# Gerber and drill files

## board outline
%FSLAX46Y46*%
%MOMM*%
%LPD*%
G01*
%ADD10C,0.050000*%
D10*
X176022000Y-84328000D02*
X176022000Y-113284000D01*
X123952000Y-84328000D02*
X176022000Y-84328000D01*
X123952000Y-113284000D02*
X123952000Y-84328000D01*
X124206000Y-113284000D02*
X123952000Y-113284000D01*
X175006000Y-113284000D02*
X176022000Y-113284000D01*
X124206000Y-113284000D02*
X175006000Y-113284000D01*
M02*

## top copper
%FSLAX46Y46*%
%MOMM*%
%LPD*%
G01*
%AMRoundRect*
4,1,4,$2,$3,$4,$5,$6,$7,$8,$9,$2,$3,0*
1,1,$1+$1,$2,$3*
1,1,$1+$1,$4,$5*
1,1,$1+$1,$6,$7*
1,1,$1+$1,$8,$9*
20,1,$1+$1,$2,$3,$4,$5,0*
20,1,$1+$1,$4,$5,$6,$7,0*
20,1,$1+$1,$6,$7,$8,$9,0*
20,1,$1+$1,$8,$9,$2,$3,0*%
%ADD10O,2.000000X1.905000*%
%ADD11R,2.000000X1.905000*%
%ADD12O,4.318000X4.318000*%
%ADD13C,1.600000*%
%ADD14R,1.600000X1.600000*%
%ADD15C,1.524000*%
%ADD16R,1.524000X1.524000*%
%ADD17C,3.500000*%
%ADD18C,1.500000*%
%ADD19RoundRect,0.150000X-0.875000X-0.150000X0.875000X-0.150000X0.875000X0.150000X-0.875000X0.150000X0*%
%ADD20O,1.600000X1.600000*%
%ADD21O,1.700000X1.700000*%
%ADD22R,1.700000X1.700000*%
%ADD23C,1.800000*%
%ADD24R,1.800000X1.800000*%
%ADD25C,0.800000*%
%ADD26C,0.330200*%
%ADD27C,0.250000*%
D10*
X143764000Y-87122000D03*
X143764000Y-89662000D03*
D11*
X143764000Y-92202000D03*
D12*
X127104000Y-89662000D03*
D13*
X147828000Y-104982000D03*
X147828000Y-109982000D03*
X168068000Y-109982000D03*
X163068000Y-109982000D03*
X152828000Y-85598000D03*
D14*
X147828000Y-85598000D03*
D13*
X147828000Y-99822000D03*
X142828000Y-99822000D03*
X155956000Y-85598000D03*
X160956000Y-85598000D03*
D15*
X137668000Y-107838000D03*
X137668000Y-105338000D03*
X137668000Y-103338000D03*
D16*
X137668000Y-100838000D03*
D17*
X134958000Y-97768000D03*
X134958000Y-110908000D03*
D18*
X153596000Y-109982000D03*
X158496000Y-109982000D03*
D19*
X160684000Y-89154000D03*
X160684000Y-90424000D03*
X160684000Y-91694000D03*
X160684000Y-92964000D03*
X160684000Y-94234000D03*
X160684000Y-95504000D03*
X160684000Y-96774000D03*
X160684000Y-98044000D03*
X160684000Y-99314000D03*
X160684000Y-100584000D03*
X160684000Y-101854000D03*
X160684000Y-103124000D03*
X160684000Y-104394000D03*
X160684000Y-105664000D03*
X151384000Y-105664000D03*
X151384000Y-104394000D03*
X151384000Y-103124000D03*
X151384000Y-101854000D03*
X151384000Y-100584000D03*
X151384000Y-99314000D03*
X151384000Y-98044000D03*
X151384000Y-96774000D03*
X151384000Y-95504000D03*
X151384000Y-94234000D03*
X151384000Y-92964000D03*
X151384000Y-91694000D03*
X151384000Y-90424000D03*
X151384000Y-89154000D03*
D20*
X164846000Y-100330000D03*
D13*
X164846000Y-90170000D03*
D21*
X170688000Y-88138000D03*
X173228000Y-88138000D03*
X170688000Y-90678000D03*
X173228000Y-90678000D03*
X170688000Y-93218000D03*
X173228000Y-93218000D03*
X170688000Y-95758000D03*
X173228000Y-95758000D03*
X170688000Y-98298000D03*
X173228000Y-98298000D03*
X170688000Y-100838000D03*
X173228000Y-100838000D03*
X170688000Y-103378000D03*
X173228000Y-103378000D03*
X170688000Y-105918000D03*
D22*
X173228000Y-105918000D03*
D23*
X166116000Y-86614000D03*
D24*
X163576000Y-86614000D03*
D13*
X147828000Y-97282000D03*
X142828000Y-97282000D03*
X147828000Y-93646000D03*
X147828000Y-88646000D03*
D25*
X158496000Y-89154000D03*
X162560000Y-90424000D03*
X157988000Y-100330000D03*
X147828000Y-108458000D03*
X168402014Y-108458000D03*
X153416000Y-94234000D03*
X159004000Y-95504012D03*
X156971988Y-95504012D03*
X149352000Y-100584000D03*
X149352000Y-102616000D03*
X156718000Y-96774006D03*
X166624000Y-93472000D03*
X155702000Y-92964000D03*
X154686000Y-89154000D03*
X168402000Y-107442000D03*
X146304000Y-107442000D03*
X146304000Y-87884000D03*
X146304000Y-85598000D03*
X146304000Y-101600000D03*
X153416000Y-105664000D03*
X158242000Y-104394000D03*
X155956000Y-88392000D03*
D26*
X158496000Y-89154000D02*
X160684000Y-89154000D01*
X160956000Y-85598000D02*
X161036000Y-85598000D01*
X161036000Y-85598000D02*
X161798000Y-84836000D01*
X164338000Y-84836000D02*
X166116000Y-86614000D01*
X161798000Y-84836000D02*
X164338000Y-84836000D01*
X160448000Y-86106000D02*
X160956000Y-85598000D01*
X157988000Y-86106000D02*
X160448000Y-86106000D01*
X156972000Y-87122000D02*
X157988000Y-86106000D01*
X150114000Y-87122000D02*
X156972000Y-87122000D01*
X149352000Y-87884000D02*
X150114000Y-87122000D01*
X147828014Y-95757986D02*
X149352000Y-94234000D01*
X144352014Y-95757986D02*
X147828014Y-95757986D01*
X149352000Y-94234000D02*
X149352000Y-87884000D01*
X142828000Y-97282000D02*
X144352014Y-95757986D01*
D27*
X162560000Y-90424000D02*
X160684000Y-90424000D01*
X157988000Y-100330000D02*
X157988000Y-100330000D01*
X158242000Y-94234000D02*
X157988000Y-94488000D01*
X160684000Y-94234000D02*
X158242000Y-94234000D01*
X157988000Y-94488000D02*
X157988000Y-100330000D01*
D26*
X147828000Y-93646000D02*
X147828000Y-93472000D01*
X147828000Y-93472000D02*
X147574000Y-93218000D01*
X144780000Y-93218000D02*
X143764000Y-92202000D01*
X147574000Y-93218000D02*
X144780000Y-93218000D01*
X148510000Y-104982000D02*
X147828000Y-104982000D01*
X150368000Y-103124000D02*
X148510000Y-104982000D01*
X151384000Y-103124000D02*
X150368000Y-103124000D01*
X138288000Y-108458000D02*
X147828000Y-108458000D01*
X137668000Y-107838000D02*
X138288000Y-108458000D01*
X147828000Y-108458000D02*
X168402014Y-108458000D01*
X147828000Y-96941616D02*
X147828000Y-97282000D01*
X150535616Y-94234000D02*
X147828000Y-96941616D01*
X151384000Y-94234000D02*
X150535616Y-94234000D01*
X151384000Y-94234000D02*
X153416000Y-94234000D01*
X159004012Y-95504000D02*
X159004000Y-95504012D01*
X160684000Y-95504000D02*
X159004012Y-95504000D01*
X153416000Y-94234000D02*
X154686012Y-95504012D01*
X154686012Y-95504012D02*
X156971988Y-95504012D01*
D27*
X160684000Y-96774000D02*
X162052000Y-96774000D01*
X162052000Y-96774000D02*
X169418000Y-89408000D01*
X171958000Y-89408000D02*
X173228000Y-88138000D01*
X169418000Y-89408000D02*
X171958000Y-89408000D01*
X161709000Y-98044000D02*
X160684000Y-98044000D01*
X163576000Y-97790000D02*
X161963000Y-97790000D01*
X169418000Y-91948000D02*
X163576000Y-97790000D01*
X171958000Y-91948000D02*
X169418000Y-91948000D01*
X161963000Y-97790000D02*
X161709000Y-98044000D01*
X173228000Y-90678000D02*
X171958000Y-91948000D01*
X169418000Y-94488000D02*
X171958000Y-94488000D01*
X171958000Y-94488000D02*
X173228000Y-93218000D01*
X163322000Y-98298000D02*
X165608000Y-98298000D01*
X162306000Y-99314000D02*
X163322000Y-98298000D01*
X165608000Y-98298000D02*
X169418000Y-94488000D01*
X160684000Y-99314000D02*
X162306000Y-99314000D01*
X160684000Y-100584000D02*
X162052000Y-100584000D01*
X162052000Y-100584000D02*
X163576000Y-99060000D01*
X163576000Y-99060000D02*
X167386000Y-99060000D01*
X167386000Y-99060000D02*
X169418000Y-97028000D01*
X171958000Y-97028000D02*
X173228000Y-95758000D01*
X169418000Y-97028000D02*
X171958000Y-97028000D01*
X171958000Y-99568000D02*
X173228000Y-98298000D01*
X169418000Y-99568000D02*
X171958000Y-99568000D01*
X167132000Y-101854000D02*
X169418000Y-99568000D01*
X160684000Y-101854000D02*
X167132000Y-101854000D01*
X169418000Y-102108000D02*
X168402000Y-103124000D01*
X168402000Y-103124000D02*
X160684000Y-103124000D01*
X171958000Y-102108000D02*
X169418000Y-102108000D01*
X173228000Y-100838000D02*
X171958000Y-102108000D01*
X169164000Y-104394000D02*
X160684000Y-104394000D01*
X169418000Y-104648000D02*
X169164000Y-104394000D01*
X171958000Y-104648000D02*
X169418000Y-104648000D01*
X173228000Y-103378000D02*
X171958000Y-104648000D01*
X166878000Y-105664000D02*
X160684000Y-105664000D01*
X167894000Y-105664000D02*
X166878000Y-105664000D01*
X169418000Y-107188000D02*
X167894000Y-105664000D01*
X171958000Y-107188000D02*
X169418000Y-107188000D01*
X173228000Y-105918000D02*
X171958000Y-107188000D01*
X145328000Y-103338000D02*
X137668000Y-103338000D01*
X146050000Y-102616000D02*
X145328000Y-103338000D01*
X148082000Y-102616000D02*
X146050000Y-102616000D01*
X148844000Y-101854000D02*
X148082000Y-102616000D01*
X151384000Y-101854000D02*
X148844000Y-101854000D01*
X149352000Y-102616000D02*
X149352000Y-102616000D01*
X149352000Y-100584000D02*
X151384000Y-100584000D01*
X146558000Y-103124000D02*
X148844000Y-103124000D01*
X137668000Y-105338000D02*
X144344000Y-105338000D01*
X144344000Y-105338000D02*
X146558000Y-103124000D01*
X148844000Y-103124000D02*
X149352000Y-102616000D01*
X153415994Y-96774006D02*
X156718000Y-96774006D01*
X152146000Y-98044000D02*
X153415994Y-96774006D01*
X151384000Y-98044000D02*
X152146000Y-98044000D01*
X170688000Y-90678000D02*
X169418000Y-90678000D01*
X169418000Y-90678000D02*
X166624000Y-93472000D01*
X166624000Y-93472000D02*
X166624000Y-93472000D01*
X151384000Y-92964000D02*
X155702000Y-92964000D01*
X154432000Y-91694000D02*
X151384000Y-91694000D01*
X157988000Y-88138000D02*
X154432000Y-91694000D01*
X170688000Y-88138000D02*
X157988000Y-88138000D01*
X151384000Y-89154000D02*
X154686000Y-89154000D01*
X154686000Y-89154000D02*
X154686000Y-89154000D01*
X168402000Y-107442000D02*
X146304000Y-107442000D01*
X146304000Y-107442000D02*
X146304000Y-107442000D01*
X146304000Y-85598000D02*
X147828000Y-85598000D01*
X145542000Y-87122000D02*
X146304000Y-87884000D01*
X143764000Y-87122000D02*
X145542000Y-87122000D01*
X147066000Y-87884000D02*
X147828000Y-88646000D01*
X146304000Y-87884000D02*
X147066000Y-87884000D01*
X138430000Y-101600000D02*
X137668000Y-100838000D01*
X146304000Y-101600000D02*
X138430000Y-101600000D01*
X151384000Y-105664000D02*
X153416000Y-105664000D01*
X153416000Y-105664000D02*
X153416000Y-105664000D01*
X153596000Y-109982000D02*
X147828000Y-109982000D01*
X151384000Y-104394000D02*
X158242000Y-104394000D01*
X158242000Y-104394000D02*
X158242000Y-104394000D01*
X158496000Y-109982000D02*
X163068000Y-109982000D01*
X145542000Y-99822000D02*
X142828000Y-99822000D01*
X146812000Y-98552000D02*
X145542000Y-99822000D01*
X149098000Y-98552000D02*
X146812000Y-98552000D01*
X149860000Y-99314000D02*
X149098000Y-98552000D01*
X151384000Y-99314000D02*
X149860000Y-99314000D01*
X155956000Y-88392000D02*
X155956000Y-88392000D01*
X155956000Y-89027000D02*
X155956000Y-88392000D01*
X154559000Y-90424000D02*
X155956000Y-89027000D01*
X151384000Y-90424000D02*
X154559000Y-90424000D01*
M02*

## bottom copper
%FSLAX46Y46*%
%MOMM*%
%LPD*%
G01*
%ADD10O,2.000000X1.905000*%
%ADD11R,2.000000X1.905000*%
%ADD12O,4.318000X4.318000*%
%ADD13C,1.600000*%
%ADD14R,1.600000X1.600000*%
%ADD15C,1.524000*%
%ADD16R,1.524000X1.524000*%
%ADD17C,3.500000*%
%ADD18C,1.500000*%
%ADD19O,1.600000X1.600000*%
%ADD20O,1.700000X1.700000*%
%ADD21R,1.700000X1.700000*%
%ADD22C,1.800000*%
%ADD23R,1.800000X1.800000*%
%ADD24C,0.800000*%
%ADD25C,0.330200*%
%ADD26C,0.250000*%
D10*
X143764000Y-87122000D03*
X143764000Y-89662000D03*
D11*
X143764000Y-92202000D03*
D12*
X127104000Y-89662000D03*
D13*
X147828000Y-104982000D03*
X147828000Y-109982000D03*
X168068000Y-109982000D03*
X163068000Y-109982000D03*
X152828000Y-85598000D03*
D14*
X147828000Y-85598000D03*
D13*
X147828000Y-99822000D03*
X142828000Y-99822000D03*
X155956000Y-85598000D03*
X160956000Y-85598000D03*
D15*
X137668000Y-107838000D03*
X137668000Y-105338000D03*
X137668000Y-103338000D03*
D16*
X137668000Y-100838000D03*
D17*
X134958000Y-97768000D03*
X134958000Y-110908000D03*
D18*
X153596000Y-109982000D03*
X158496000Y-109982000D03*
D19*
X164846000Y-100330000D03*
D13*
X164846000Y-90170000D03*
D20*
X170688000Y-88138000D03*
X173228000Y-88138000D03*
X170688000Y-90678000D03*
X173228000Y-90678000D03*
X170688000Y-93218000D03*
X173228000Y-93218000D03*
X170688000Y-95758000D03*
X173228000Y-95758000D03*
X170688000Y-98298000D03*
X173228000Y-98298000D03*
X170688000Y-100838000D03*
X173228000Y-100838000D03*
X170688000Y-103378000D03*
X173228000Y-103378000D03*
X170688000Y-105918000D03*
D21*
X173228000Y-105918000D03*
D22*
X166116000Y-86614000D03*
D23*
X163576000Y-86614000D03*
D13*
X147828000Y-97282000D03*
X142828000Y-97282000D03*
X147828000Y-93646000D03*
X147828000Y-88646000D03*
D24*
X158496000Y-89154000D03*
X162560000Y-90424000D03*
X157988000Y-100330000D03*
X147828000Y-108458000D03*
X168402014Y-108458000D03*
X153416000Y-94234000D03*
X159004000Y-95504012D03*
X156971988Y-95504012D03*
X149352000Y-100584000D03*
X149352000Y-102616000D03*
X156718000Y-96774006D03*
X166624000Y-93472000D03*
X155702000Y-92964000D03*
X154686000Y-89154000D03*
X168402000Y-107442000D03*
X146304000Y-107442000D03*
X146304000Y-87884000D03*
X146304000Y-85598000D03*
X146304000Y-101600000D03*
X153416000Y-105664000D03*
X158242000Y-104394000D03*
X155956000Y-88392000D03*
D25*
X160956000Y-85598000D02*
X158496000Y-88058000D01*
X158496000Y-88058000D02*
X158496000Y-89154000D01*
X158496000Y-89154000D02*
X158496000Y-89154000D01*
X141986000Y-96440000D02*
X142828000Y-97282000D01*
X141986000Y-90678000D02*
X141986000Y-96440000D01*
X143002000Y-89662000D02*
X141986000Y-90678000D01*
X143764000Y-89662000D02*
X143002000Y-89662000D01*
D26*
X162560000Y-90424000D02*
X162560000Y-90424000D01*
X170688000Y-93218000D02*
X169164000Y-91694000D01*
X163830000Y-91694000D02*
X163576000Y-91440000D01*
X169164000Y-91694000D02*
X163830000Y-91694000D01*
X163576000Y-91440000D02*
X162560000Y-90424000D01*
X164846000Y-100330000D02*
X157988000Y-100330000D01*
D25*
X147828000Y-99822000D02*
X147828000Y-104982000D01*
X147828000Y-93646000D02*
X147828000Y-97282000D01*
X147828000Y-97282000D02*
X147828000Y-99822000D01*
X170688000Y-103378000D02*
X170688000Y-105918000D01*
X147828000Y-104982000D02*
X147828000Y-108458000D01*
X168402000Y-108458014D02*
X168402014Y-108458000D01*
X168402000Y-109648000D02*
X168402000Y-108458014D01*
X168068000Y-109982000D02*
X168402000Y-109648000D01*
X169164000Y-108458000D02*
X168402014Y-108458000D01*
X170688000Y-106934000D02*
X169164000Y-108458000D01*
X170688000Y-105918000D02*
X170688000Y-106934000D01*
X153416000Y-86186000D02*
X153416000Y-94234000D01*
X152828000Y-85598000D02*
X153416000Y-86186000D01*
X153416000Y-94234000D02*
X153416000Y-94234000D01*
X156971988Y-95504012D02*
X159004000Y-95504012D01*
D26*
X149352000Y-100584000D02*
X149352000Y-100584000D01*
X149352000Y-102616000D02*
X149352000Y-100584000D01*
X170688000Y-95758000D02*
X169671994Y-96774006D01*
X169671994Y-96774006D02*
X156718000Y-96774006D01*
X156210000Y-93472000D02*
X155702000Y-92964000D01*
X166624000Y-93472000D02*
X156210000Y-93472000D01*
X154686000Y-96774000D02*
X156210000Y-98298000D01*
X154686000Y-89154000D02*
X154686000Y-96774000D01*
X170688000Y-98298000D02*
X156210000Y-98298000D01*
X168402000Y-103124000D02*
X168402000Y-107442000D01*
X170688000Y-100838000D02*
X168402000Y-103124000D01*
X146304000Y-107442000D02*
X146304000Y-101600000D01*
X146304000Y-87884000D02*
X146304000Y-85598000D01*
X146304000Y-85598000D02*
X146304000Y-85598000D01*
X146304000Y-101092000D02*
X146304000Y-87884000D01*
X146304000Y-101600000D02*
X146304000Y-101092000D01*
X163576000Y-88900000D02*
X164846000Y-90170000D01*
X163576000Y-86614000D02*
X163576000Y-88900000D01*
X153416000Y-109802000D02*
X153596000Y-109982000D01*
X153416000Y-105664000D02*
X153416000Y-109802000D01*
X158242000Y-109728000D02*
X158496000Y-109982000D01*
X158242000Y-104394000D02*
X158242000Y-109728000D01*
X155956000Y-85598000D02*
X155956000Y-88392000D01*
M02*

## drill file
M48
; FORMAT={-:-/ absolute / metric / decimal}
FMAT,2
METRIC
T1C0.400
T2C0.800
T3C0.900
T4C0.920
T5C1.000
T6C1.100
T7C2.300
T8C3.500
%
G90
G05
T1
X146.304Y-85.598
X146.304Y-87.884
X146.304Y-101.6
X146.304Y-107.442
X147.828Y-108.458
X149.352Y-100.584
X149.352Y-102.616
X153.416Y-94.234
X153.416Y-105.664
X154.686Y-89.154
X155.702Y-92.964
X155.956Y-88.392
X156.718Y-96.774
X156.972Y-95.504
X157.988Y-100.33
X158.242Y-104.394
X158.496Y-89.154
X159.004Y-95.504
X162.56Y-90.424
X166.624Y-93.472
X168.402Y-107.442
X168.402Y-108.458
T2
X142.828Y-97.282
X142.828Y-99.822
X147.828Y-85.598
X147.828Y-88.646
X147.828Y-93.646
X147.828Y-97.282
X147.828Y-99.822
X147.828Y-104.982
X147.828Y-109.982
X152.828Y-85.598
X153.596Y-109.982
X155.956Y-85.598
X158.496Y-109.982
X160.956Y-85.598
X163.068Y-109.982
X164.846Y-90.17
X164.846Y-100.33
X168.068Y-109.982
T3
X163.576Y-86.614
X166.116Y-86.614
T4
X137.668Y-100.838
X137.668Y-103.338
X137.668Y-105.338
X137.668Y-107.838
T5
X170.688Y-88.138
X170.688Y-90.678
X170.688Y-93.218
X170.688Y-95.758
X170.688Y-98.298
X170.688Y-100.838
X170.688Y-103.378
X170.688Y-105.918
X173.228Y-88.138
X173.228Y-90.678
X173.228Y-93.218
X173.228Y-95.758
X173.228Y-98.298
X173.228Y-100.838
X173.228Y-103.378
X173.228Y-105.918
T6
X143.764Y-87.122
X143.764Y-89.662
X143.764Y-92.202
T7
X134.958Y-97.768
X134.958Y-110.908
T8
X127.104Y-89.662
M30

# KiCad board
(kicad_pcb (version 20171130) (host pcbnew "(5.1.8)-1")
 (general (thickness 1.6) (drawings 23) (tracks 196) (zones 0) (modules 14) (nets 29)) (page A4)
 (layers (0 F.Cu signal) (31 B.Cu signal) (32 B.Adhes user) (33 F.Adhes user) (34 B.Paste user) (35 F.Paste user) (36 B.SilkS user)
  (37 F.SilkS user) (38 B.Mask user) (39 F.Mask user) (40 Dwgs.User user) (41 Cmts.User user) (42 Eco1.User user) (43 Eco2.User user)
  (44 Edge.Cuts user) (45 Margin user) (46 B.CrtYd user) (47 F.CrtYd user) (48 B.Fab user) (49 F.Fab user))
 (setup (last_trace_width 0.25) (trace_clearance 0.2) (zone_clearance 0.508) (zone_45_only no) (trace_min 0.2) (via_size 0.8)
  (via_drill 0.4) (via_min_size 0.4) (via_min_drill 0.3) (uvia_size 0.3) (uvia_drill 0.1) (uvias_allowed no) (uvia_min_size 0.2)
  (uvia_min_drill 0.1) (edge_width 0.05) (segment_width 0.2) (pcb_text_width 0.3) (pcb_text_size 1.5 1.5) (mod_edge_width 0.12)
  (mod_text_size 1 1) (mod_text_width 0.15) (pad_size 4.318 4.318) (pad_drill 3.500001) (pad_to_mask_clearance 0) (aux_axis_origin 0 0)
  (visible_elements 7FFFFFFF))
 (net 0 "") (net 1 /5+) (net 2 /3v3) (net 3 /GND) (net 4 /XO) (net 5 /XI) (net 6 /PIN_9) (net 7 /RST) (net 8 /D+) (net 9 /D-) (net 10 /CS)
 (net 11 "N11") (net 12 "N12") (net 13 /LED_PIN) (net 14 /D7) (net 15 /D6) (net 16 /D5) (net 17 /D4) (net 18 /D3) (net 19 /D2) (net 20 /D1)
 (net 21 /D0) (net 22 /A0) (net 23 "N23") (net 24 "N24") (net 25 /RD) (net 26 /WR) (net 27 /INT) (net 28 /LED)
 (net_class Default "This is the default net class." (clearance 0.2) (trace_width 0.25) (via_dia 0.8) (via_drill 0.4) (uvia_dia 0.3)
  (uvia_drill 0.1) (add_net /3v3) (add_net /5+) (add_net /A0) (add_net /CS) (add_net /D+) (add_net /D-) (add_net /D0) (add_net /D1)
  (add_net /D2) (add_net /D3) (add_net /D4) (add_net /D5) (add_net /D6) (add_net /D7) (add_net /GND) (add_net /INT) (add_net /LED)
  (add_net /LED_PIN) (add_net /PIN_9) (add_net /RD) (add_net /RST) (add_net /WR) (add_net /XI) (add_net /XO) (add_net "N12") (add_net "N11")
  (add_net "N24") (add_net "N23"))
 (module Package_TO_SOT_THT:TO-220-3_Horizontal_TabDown (layer F.Cu) (at 143.764 92.202 90)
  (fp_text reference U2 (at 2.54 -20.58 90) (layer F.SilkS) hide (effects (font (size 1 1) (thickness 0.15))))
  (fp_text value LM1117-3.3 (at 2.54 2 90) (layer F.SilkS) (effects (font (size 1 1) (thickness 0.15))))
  (pad 3 thru_hole oval (at 5.08 0 90) (size 1.905 2) (drill 1.1) (layers *.Cu *.Mask) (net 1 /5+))
  (pad 2 thru_hole oval (at 2.54 0 90) (size 1.905 2) (drill 1.1) (layers *.Cu *.Mask) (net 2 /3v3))
  (pad 1 thru_hole rect (at 0 0 90) (size 1.905 2) (drill 1.1) (layers *.Cu *.Mask) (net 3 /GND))
  (pad "" thru_hole oval (at 2.54 -16.66 90) (size 4.318 4.318) (drill 3.500001) (layers *.Cu *.Mask)))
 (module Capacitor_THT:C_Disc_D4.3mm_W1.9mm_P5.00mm (layer F.Cu) (at 147.828 109.982 90)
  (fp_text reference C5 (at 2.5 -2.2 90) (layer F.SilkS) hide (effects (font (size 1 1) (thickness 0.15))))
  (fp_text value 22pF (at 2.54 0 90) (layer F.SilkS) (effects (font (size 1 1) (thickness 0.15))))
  (pad 2 thru_hole circle (at 5 0 90) (size 1.6 1.6) (drill 0.8) (layers *.Cu *.Mask) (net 3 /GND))
  (pad 1 thru_hole circle (at 0 0 90) (size 1.6 1.6) (drill 0.8) (layers *.Cu *.Mask) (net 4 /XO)))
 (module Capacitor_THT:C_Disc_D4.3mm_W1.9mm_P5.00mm (layer F.Cu) (at 163.068 109.982)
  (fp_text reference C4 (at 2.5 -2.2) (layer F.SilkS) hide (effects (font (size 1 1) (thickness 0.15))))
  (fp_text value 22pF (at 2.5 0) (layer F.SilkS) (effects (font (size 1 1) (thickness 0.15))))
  (pad 2 thru_hole circle (at 5 0) (size 1.6 1.6) (drill 0.8) (layers *.Cu *.Mask) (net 3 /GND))
  (pad 1 thru_hole circle (at 0 0) (size 1.6 1.6) (drill 0.8) (layers *.Cu *.Mask) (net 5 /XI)))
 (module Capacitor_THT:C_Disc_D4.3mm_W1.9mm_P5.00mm (layer F.Cu) (at 147.828 85.598)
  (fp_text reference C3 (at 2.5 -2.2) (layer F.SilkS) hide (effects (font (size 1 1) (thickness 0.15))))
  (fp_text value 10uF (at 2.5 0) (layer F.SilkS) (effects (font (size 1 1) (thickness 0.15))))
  (pad 2 thru_hole circle (at 5 0) (size 1.6 1.6) (drill 0.8) (layers *.Cu *.Mask) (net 3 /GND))
  (pad 1 thru_hole rect (at 0 0) (size 1.6 1.6) (drill 0.8) (layers *.Cu *.Mask) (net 1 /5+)))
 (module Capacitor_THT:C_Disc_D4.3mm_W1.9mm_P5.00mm (layer F.Cu) (at 142.828 99.822)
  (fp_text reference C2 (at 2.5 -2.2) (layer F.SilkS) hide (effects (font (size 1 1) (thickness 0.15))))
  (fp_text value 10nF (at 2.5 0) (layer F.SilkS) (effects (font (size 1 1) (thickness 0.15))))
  (pad 2 thru_hole circle (at 5 0) (size 1.6 1.6) (drill 0.8) (layers *.Cu *.Mask) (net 3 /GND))
  (pad 1 thru_hole circle (at 0 0) (size 1.6 1.6) (drill 0.8) (layers *.Cu *.Mask) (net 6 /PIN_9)))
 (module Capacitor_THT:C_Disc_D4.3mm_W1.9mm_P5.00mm (layer F.Cu) (at 160.956 85.598 180)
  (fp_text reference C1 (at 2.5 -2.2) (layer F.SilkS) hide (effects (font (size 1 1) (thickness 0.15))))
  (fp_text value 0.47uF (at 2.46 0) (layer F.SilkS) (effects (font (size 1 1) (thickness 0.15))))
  (pad 2 thru_hole circle (at 5 0 180) (size 1.6 1.6) (drill 0.8) (layers *.Cu *.Mask) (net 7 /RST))
  (pad 1 thru_hole circle (at 0 0 180) (size 1.6 1.6) (drill 0.8) (layers *.Cu *.Mask) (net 2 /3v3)))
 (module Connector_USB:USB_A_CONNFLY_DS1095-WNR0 (layer F.Cu) (at 137.668 100.838 270)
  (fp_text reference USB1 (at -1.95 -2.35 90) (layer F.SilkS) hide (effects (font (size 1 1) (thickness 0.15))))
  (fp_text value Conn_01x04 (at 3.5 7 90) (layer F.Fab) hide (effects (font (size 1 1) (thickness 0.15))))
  (pad 4 thru_hole circle (at 7 0 270) (size 1.524 1.524) (drill 0.92) (layers *.Cu *.Mask) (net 3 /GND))
  (pad 3 thru_hole circle (at 4.5 0 270) (size 1.524 1.524) (drill 0.92) (layers *.Cu *.Mask) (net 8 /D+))
  (pad 2 thru_hole circle (at 2.5 0 270) (size 1.524 1.524) (drill 0.92) (layers *.Cu *.Mask) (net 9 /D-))
  (pad 1 thru_hole rect (at 0 0 270) (size 1.524 1.524) (drill 0.92) (layers *.Cu *.Mask) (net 1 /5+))
  (pad 5 thru_hole circle (at -3.07 2.71 270) (size 3.5 3.5) (drill 2.3) (layers *.Cu *.Mask))
  (pad 5 thru_hole circle (at 10.07 2.71 270) (size 3.5 3.5) (drill 2.3) (layers *.Cu *.Mask)))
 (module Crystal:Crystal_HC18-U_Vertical (layer F.Cu) (at 158.496 109.982 180)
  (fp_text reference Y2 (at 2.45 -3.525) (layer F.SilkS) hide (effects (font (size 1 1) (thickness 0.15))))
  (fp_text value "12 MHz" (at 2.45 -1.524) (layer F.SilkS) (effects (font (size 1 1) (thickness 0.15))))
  (pad 2 thru_hole circle (at 4.9 0 180) (size 1.5 1.5) (drill 0.8) (layers *.Cu *.Mask) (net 4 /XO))
  (pad 1 thru_hole circle (at 0 0 180) (size 1.5 1.5) (drill 0.8) (layers *.Cu *.Mask) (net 5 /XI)))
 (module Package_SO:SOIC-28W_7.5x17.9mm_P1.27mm (layer F.Cu) (at 156.034 97.409)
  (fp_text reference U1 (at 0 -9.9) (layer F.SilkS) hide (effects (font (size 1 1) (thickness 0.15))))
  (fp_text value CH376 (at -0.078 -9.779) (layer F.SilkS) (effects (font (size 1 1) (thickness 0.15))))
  (pad 28 smd roundrect (at 4.65 -8.255) (size 2.05 0.6) (layers F.Cu F.Paste F.Mask) (roundrect_rratio 0.25) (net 2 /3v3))
  (pad 27 smd roundrect (at 4.65 -6.985) (size 2.05 0.6) (layers F.Cu F.Paste F.Mask) (roundrect_rratio 0.25) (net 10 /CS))
  (pad 26 smd roundrect (at 4.65 -5.715) (size 2.05 0.6) (layers F.Cu F.Paste F.Mask) (roundrect_rratio 0.25) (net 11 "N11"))
  (pad 25 smd roundrect (at 4.65 -4.445) (size 2.05 0.6) (layers F.Cu F.Paste F.Mask) (roundrect_rratio 0.25) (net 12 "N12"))
  (pad 24 smd roundrect (at 4.65 -3.175) (size 2.05 0.6) (layers F.Cu F.Paste F.Mask) (roundrect_rratio 0.25) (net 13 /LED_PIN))
  (pad 23 smd roundrect (at 4.65 -1.905) (size 2.05 0.6) (layers F.Cu F.Paste F.Mask) (roundrect_rratio 0.25) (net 3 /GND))
  (pad 22 smd roundrect (at 4.65 -0.635) (size 2.05 0.6) (layers F.Cu F.Paste F.Mask) (roundrect_rratio 0.25) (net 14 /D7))
  (pad 21 smd roundrect (at 4.65 0.635) (size 2.05 0.6) (layers F.Cu F.Paste F.Mask) (roundrect_rratio 0.25) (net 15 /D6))
  (pad 20 smd roundrect (at 4.65 1.905) (size 2.05 0.6) (layers F.Cu F.Paste F.Mask) (roundrect_rratio 0.25) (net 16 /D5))
  (pad 19 smd roundrect (at 4.65 3.175) (size 2.05 0.6) (layers F.Cu F.Paste F.Mask) (roundrect_rratio 0.25) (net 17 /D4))
  (pad 18 smd roundrect (at 4.65 4.445) (size 2.05 0.6) (layers F.Cu F.Paste F.Mask) (roundrect_rratio 0.25) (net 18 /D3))
  (pad 17 smd roundrect (at 4.65 5.715) (size 2.05 0.6) (layers F.Cu F.Paste F.Mask) (roundrect_rratio 0.25) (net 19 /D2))
  (pad 16 smd roundrect (at 4.65 6.985) (size 2.05 0.6) (layers F.Cu F.Paste F.Mask) (roundrect_rratio 0.25) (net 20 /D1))
  (pad 15 smd roundrect (at 4.65 8.255) (size 2.05 0.6) (layers F.Cu F.Paste F.Mask) (roundrect_rratio 0.25) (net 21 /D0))
  (pad 14 smd roundrect (at -4.65 8.255) (size 2.05 0.6) (layers F.Cu F.Paste F.Mask) (roundrect_rratio 0.25) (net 4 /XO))
  (pad 13 smd roundrect (at -4.65 6.985) (size 2.05 0.6) (layers F.Cu F.Paste F.Mask) (roundrect_rratio 0.25) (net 5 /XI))
  (pad 12 smd roundrect (at -4.65 5.715) (size 2.05 0.6) (layers F.Cu F.Paste F.Mask) (roundrect_rratio 0.25) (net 3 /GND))
  (pad 11 smd roundrect (at -4.65 4.445) (size 2.05 0.6) (layers F.Cu F.Paste F.Mask) (roundrect_rratio 0.25) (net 9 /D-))
  (pad 10 smd roundrect (at -4.65 3.175) (size 2.05 0.6) (layers F.Cu F.Paste F.Mask) (roundrect_rratio 0.25) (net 8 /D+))
  (pad 9 smd roundrect (at -4.65 1.905) (size 2.05 0.6) (layers F.Cu F.Paste F.Mask) (roundrect_rratio 0.25) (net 6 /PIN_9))
  (pad 8 smd roundrect (at -4.65 0.635) (size 2.05 0.6) (layers F.Cu F.Paste F.Mask) (roundrect_rratio 0.25) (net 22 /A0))
  (pad 7 smd roundrect (at -4.65 -0.635) (size 2.05 0.6) (layers F.Cu F.Paste F.Mask) (roundrect_rratio 0.25) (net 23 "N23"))
  (pad 6 smd roundrect (at -4.65 -1.905) (size 2.05 0.6) (layers F.Cu F.Paste F.Mask) (roundrect_rratio 0.25) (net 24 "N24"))
  (pad 5 smd roundrect (at -4.65 -3.175) (size 2.05 0.6) (layers F.Cu F.Paste F.Mask) (roundrect_rratio 0.25) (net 3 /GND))
  (pad 4 smd roundrect (at -4.65 -4.445) (size 2.05 0.6) (layers F.Cu F.Paste F.Mask) (roundrect_rratio 0.25) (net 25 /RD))
  (pad 3 smd roundrect (at -4.65 -5.715) (size 2.05 0.6) (layers F.Cu F.Paste F.Mask) (roundrect_rratio 0.25) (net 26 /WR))
  (pad 2 smd roundrect (at -4.65 -6.985) (size 2.05 0.6) (layers F.Cu F.Paste F.Mask) (roundrect_rratio 0.25) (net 7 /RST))
  (pad 1 smd roundrect (at -4.65 -8.255) (size 2.05 0.6) (layers F.Cu F.Paste F.Mask) (roundrect_rratio 0.25) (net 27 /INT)))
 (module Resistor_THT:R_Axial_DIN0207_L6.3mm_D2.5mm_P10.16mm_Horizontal (layer F.Cu) (at 164.846 90.17 270)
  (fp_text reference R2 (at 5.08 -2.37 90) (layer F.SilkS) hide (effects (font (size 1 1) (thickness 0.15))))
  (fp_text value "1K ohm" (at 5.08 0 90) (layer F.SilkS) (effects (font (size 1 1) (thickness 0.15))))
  (pad 2 thru_hole oval (at 10.16 0 270) (size 1.6 1.6) (drill 0.8) (layers *.Cu *.Mask) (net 13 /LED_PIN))
  (pad 1 thru_hole circle (at 0 0 270) (size 1.6 1.6) (drill 0.8) (layers *.Cu *.Mask) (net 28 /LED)))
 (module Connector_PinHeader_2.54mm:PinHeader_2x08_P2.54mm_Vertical (layer F.Cu) (at 173.228 105.918 180)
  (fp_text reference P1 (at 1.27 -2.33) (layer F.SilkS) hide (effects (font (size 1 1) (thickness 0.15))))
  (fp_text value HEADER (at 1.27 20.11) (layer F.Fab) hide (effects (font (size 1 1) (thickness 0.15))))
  (pad 16 thru_hole oval (at 2.54 17.78 180) (size 1.7 1.7) (drill 1) (layers *.Cu *.Mask) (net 26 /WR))
  (pad 15 thru_hole oval (at 0 17.78 180) (size 1.7 1.7) (drill 1) (layers *.Cu *.Mask) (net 14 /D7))
  (pad 14 thru_hole oval (at 2.54 15.24 180) (size 1.7 1.7) (drill 1) (layers *.Cu *.Mask) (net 25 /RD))
  (pad 13 thru_hole oval (at 0 15.24 180) (size 1.7 1.7) (drill 1) (layers *.Cu *.Mask) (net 15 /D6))
  (pad 12 thru_hole oval (at 2.54 12.7 180) (size 1.7 1.7) (drill 1) (layers *.Cu *.Mask) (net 10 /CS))
  (pad 11 thru_hole oval (at 0 12.7 180) (size 1.7 1.7) (drill 1) (layers *.Cu *.Mask) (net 16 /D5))
  (pad 10 thru_hole oval (at 2.54 10.16 180) (size 1.7 1.7) (drill 1) (layers *.Cu *.Mask) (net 22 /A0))
  (pad 9 thru_hole oval (at 0 10.16 180) (size 1.7 1.7) (drill 1) (layers *.Cu *.Mask) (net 17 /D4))
  (pad 8 thru_hole oval (at 2.54 7.62 180) (size 1.7 1.7) (drill 1) (layers *.Cu *.Mask) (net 27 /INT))
  (pad 7 thru_hole oval (at 0 7.62 180) (size 1.7 1.7) (drill 1) (layers *.Cu *.Mask) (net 18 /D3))
  (pad 6 thru_hole oval (at 2.54 5.08 180) (size 1.7 1.7) (drill 1) (layers *.Cu *.Mask) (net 1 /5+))
  (pad 5 thru_hole oval (at 0 5.08 180) (size 1.7 1.7) (drill 1) (layers *.Cu *.Mask) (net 19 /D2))
  (pad 4 thru_hole oval (at 2.54 2.54 180) (size 1.7 1.7) (drill 1) (layers *.Cu *.Mask) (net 3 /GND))
  (pad 3 thru_hole oval (at 0 2.54 180) (size 1.7 1.7) (drill 1) (layers *.Cu *.Mask) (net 20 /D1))
  (pad 2 thru_hole oval (at 2.54 0 180) (size 1.7 1.7) (drill 1) (layers *.Cu *.Mask) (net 3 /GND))
  (pad 1 thru_hole rect (at 0 0 180) (size 1.7 1.7) (drill 1) (layers *.Cu *.Mask) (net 21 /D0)))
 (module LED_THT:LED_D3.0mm (layer F.Cu) (at 163.576 86.614)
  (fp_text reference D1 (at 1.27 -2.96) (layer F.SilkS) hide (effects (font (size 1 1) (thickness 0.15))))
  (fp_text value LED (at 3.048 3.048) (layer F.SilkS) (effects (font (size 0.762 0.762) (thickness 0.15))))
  (pad 2 thru_hole circle (at 2.54 0) (size 1.8 1.8) (drill 0.9) (layers *.Cu *.Mask) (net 2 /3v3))
  (pad 1 thru_hole rect (at 0 0) (size 1.8 1.8) (drill 0.9) (layers *.Cu *.Mask) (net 28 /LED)))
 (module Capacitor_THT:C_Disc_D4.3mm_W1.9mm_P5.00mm (layer F.Cu) (at 142.828 97.282)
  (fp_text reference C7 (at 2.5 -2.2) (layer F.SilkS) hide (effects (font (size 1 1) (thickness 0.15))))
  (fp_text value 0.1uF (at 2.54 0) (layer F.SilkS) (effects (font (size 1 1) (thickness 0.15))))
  (pad 2 thru_hole circle (at 5 0) (size 1.6 1.6) (drill 0.8) (layers *.Cu *.Mask) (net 3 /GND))
  (pad 1 thru_hole circle (at 0 0) (size 1.6 1.6) (drill 0.8) (layers *.Cu *.Mask) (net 2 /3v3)))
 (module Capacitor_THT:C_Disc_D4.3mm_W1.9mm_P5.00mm (layer F.Cu) (at 147.828 88.646 270)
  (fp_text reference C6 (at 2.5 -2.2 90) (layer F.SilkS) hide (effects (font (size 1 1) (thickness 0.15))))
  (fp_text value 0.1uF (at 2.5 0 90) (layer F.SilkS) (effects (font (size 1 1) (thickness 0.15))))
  (pad 2 thru_hole circle (at 5 0 270) (size 1.6 1.6) (drill 0.8) (layers *.Cu *.Mask) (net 3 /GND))
  (pad 1 thru_hole circle (at 0 0 270) (size 1.6 1.6) (drill 0.8) (layers *.Cu *.Mask) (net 1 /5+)))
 (gr_line (start 176.022 84.328) (end 176.022 113.284) (layer Edge.Cuts) (width 0.05))
 (gr_line (start 123.952 84.328) (end 176.022 84.328) (layer Edge.Cuts) (width 0.05))
 (gr_line (start 123.952 113.284) (end 123.952 84.328) (layer Edge.Cuts) (width 0.05))
 (gr_line (start 124.206 113.284) (end 123.952 113.284) (layer Edge.Cuts) (width 0.05))
 (gr_line (start 175.006 113.284) (end 176.022 113.284) (layer Edge.Cuts) (width 0.05))
 (gr_line (start 124.206 113.284) (end 175.006 113.284) (layer Edge.Cuts) (width 0.05))
 (segment (start 160.956 85.598) (end 158.496 88.058) (width 0.3302) (layer B.Cu) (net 2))
 (segment (start 158.496 88.058) (end 158.496 89.154) (width 0.3302) (layer B.Cu) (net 2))
 (segment (start 158.496 89.154) (end 158.496 89.154) (width 0.3302) (layer B.Cu) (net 2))
 (via (at 158.496 89.154) (size 0.8) (drill 0.4) (layers F.Cu B.Cu) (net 2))
 (segment (start 158.496 89.154) (end 160.684 89.154) (width 0.3302) (layer F.Cu) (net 2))
 (segment (start 160.956 85.598) (end 161.036 85.598) (width 0.3302) (layer F.Cu) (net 2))
 (segment (start 161.036 85.598) (end 161.798 84.836) (width 0.3302) (layer F.Cu) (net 2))
 (segment (start 164.338 84.836) (end 166.116 86.614) (width 0.3302) (layer F.Cu) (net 2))
 (segment (start 161.798 84.836) (end 164.338 84.836) (width 0.3302) (layer F.Cu) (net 2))
 (segment (start 141.986 96.44) (end 142.828 97.282) (width 0.3302) (layer B.Cu) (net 2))
 (segment (start 141.986 90.678) (end 141.986 96.44) (width 0.3302) (layer B.Cu) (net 2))
 (segment (start 143.002 89.662) (end 141.986 90.678) (width 0.3302) (layer B.Cu) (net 2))
 (segment (start 143.764 89.662) (end 143.002 89.662) (width 0.3302) (layer B.Cu) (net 2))
 (segment (start 160.448 86.106) (end 160.956 85.598) (width 0.3302) (layer F.Cu) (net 2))
 (segment (start 157.988 86.106) (end 160.448 86.106) (width 0.3302) (layer F.Cu) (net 2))
 (segment (start 156.972 87.122) (end 157.988 86.106) (width 0.3302) (layer F.Cu) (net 2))
 (segment (start 150.114 87.122) (end 156.972 87.122) (width 0.3302) (layer F.Cu) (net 2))
 (segment (start 149.352 87.884) (end 150.114 87.122) (width 0.3302) (layer F.Cu) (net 2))
 (segment (start 147.828014 95.757986) (end 149.352 94.234) (width 0.3302) (layer F.Cu) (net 2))
 (segment (start 144.352014 95.757986) (end 147.828014 95.757986) (width 0.3302) (layer F.Cu) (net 2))
 (segment (start 149.352 94.234) (end 149.352 87.884) (width 0.3302) (layer F.Cu) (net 2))
 (segment (start 142.828 97.282) (end 144.352014 95.757986) (width 0.3302) (layer F.Cu) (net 2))
 (segment (start 162.56 90.424) (end 162.56 90.424) (width 0.25) (layer B.Cu) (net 10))
 (via (at 162.56 90.424) (size 0.8) (drill 0.4) (layers F.Cu B.Cu) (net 10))
 (segment (start 162.56 90.424) (end 160.684 90.424) (width 0.25) (layer F.Cu) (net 10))
 (segment (start 170.688 93.218) (end 169.164 91.694) (width 0.25) (layer B.Cu) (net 10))
 (segment (start 163.83 91.694) (end 163.576 91.44) (width 0.25) (layer B.Cu) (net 10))
 (segment (start 169.164 91.694) (end 163.83 91.694) (width 0.25) (layer B.Cu) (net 10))
 (segment (start 163.576 91.44) (end 162.56 90.424) (width 0.25) (layer B.Cu) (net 10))
 (segment (start 157.988 100.33) (end 157.988 100.33) (width 0.25) (layer F.Cu) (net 13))
 (via (at 157.988 100.33) (size 0.8) (drill 0.4) (layers F.Cu B.Cu) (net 13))
 (segment (start 164.846 100.33) (end 157.988 100.33) (width 0.25) (layer B.Cu) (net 13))
 (segment (start 158.242 94.234) (end 157.988 94.488) (width 0.25) (layer F.Cu) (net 13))
 (segment (start 160.684 94.234) (end 158.242 94.234) (width 0.25) (layer F.Cu) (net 13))
 (segment (start 157.988 94.488) (end 157.988 100.33) (width 0.25) (layer F.Cu) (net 13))
 (segment (start 147.828 99.822) (end 147.828 104.982) (width 0.3302) (layer B.Cu) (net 3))
 (segment (start 147.828 93.646) (end 147.828 97.282) (width 0.3302) (layer B.Cu) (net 3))
 (segment (start 147.828 97.282) (end 147.828 99.822) (width 0.3302) (layer B.Cu) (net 3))
 (segment (start 147.828 93.646) (end 147.828 93.472) (width 0.3302) (layer F.Cu) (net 3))
 (segment (start 147.828 93.472) (end 147.574 93.218) (width 0.3302) (layer F.Cu) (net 3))
 (segment (start 144.78 93.218) (end 143.764 92.202) (width 0.3302) (layer F.Cu) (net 3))
 (segment (start 147.574 93.218) (end 144.78 93.218) (width 0.3302) (layer F.Cu) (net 3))
 (segment (start 148.51 104.982) (end 147.828 104.982) (width 0.3302) (layer F.Cu) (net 3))
 (segment (start 150.368 103.124) (end 148.51 104.982) (width 0.3302) (layer F.Cu) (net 3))
 (segment (start 151.384 103.124) (end 150.368 103.124) (width 0.3302) (layer F.Cu) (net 3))
 (segment (start 170.688 103.378) (end 170.688 105.918) (width 0.3302) (layer B.Cu) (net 3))
 (via (at 147.828 108.458) (size 0.8) (drill 0.4) (layers F.Cu B.Cu) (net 3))
 (segment (start 147.828 104.982) (end 147.828 108.458) (width 0.3302) (layer B.Cu) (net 3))
 (segment (start 138.288 108.458) (end 147.828 108.458) (width 0.3302) (layer F.Cu) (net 3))
 (segment (start 137.668 107.838) (end 138.288 108.458) (width 0.3302) (layer F.Cu) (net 3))
 (via (at 168.402014 108.458) (size 0.8) (drill 0.4) (layers F.Cu B.Cu) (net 3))
 (segment (start 147.828 108.458) (end 168.402014 108.458) (width 0.3302) (layer F.Cu) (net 3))
 (segment (start 168.402 108.458014) (end 168.402014 108.458) (width 0.3302) (layer B.Cu) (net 3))
 (segment (start 168.402 109.648) (end 168.402 108.458014) (width 0.3302) (layer B.Cu) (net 3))
 (segment (start 168.068 109.982) (end 168.402 109.648) (width 0.3302) (layer B.Cu) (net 3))
 (segment (start 169.164 108.458) (end 168.402014 108.458) (width 0.3302) (layer B.Cu) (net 3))
 (segment (start 170.688 106.934) (end 169.164 108.458) (width 0.3302) (layer B.Cu) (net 3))
 (segment (start 170.688 105.918) (end 170.688 106.934) (width 0.3302) (layer B.Cu) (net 3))
 (segment (start 147.828 96.941616) (end 147.828 97.282) (width 0.3302) (layer F.Cu) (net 3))
 (segment (start 150.535616 94.234) (end 147.828 96.941616) (width 0.3302) (layer F.Cu) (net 3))
 (segment (start 151.384 94.234) (end 150.535616 94.234) (width 0.3302) (layer F.Cu) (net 3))
 (segment (start 153.416 86.186) (end 153.416 94.234) (width 0.3302) (layer B.Cu) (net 3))
 (segment (start 152.828 85.598) (end 153.416 86.186) (width 0.3302) (layer B.Cu) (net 3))
 (segment (start 153.416 94.234) (end 153.416 94.234) (width 0.3302) (layer B.Cu) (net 3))
 (via (at 153.416 94.234) (size 0.8) (drill 0.4) (layers F.Cu B.Cu) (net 3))
 (segment (start 151.384 94.234) (end 153.416 94.234) (width 0.3302) (layer F.Cu) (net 3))
 (via (at 159.004 95.504012) (size 0.8) (drill 0.4) (layers F.Cu B.Cu) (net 3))
 (segment (start 159.004012 95.504) (end 159.004 95.504012) (width 0.3302) (layer F.Cu) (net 3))
 (segment (start 160.684 95.504) (end 159.004012 95.504) (width 0.3302) (layer F.Cu) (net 3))
 (segment (start 153.416 94.234) (end 154.686012 95.504012) (width 0.3302) (layer F.Cu) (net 3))
 (segment (start 154.686012 95.504012) (end 156.971988 95.504012) (width 0.3302) (layer F.Cu) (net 3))
 (via (at 156.971988 95.504012) (size 0.8) (drill 0.4) (layers F.Cu B.Cu) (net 3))
 (segment (start 156.971988 95.504012) (end 159.004 95.504012) (width 0.3302) (layer B.Cu) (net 3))
 (segment (start 160.684 96.774) (end 162.052 96.774) (width 0.25) (layer F.Cu) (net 14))
 (segment (start 162.052 96.774) (end 169.418 89.408) (width 0.25) (layer F.Cu) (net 14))
 (segment (start 171.958 89.408) (end 173.228 88.138) (width 0.25) (layer F.Cu) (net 14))
 (segment (start 169.418 89.408) (end 171.958 89.408) (width 0.25) (layer F.Cu) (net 14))
 (segment (start 161.709 98.044) (end 160.684 98.044) (width 0.25) (layer F.Cu) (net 15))
 (segment (start 163.576 97.79) (end 161.963 97.79) (width 0.25) (layer F.Cu) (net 15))
 (segment (start 169.418 91.948) (end 163.576 97.79) (width 0.25) (layer F.Cu) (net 15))
 (segment (start 171.958 91.948) (end 169.418 91.948) (width 0.25) (layer F.Cu) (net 15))
 (segment (start 161.963 97.79) (end 161.709 98.044) (width 0.25) (layer F.Cu) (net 15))
 (segment (start 173.228 90.678) (end 171.958 91.948) (width 0.25) (layer F.Cu) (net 15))
 (segment (start 169.418 94.488) (end 171.958 94.488) (width 0.25) (layer F.Cu) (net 16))
 (segment (start 171.958 94.488) (end 173.228 93.218) (width 0.25) (layer F.Cu) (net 16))
 (segment (start 163.322 98.298) (end 165.608 98.298) (width 0.25) (layer F.Cu) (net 16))
 (segment (start 162.306 99.314) (end 163.322 98.298) (width 0.25) (layer F.Cu) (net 16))
 (segment (start 165.608 98.298) (end 169.418 94.488) (width 0.25) (layer F.Cu) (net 16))
 (segment (start 160.684 99.314) (end 162.306 99.314) (width 0.25) (layer F.Cu) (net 16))
 (segment (start 160.684 100.584) (end 162.052 100.584) (width 0.25) (layer F.Cu) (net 17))
 (segment (start 162.052 100.584) (end 163.576 99.06) (width 0.25) (layer F.Cu) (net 17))
 (segment (start 163.576 99.06) (end 167.386 99.06) (width 0.25) (layer F.Cu) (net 17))
 (segment (start 167.386 99.06) (end 169.418 97.028) (width 0.25) (layer F.Cu) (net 17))
 (segment (start 171.958 97.028) (end 173.228 95.758) (width 0.25) (layer F.Cu) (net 17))
 (segment (start 169.418 97.028) (end 171.958 97.028) (width 0.25) (layer F.Cu) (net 17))
 (segment (start 171.958 99.568) (end 173.228 98.298) (width 0.25) (layer F.Cu) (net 18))
 (segment (start 169.418 99.568) (end 171.958 99.568) (width 0.25) (layer F.Cu) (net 18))
 (segment (start 167.132 101.854) (end 169.418 99.568) (width 0.25) (layer F.Cu) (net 18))
 (segment (start 160.684 101.854) (end 167.132 101.854) (width 0.25) (layer F.Cu) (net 18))
 (segment (start 169.418 102.108) (end 168.402 103.124) (width 0.25) (layer F.Cu) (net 19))
 (segment (start 168.402 103.124) (end 160.684 103.124) (width 0.25) (layer F.Cu) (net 19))
 (segment (start 171.958 102.108) (end 169.418 102.108) (width 0.25) (layer F.Cu) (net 19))
 (segment (start 173.228 100.838) (end 171.958 102.108) (width 0.25) (layer F.Cu) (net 19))
 (segment (start 169.164 104.394) (end 160.684 104.394) (width 0.25) (layer F.Cu) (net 20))
 (segment (start 169.418 104.648) (end 169.164 104.394) (width 0.25) (layer F.Cu) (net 20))
 (segment (start 171.958 104.648) (end 169.418 104.648) (width 0.25) (layer F.Cu) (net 20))
 (segment (start 173.228 103.378) (end 171.958 104.648) (width 0.25) (layer F.Cu) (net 20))
 (segment (start 166.878 105.664) (end 160.684 105.664) (width 0.25) (layer F.Cu) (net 21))
 (segment (start 167.894 105.664) (end 166.878 105.664) (width 0.25) (layer F.Cu) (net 21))
 (segment (start 169.418 107.188) (end 167.894 105.664) (width 0.25) (layer F.Cu) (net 21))
 (segment (start 171.958 107.188) (end 169.418 107.188) (width 0.25) (layer F.Cu) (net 21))
 (segment (start 173.228 105.918) (end 171.958 107.188) (width 0.25) (layer F.Cu) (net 21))
 (segment (start 145.328 103.338) (end 137.668 103.338) (width 0.25) (layer F.Cu) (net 9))
 (segment (start 146.05 102.616) (end 145.328 103.338) (width 0.25) (layer F.Cu) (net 9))
 (segment (start 148.082 102.616) (end 146.05 102.616) (width 0.25) (layer F.Cu) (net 9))
 (segment (start 148.844 101.854) (end 148.082 102.616) (width 0.25) (layer F.Cu) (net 9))
 (segment (start 151.384 101.854) (end 148.844 101.854) (width 0.25) (layer F.Cu) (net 9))
 (segment (start 149.352 102.616) (end 149.352 102.616) (width 0.25) (layer F.Cu) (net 8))
 (segment (start 149.352 100.584) (end 149.352 100.584) (width 0.25) (layer B.Cu) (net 8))
 (via (at 149.352 100.584) (size 0.8) (drill 0.4) (layers F.Cu B.Cu) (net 8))
 (segment (start 149.352 100.584) (end 151.384 100.584) (width 0.25) (layer F.Cu) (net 8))
 (segment (start 146.558 103.124) (end 148.844 103.124) (width 0.25) (layer F.Cu) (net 8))
 (via (at 149.352 102.616) (size 0.8) (drill 0.4) (layers F.Cu B.Cu) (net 8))
 (segment (start 149.352 102.616) (end 149.352 100.584) (width 0.25) (layer B.Cu) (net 8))
 (segment (start 137.668 105.338) (end 144.344 105.338) (width 0.25) (layer F.Cu) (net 8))
 (segment (start 144.344 105.338) (end 146.558 103.124) (width 0.25) (layer F.Cu) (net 8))
 (segment (start 148.844 103.124) (end 149.352 102.616) (width 0.25) (layer F.Cu) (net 8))
 (via (at 156.718 96.774006) (size 0.8) (drill 0.4) (layers F.Cu B.Cu) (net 22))
 (segment (start 170.688 95.758) (end 169.671994 96.774006) (width 0.25) (layer B.Cu) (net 22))
 (segment (start 169.671994 96.774006) (end 156.718 96.774006) (width 0.25) (layer B.Cu) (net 22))
 (segment (start 153.415994 96.774006) (end 156.718 96.774006) (width 0.25) (layer F.Cu) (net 22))
 (segment (start 152.146 98.044) (end 153.415994 96.774006) (width 0.25) (layer F.Cu) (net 22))
 (segment (start 151.384 98.044) (end 152.146 98.044) (width 0.25) (layer F.Cu) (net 22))
 (segment (start 170.688 90.678) (end 169.418 90.678) (width 0.25) (layer F.Cu) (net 25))
 (segment (start 169.418 90.678) (end 166.624 93.472) (width 0.25) (layer F.Cu) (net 25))
 (segment (start 166.624 93.472) (end 166.624 93.472) (width 0.25) (layer F.Cu) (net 25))
 (via (at 166.624 93.472) (size 0.8) (drill 0.4) (layers F.Cu B.Cu) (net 25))
 (segment (start 156.21 93.472) (end 155.702 92.964) (width 0.25) (layer B.Cu) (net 25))
 (segment (start 166.624 93.472) (end 156.21 93.472) (width 0.25) (layer B.Cu) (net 25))
 (segment (start 151.384 92.964) (end 155.702 92.964) (width 0.25) (layer F.Cu) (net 25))
 (via (at 155.702 92.964) (size 0.8) (drill 0.4) (layers F.Cu B.Cu) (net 25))
 (segment (start 154.432 91.694) (end 151.384 91.694) (width 0.25) (layer F.Cu) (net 26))
 (segment (start 157.988 88.138) (end 154.432 91.694) (width 0.25) (layer F.Cu) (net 26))
 (segment (start 170.688 88.138) (end 157.988 88.138) (width 0.25) (layer F.Cu) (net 26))
 (segment (start 151.384 89.154) (end 154.686 89.154) (width 0.25) (layer F.Cu) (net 27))
 (segment (start 154.686 89.154) (end 154.686 89.154) (width 0.25) (layer F.Cu) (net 27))
 (via (at 154.686 89.154) (size 0.8) (drill 0.4) (layers F.Cu B.Cu) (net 27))
 (segment (start 154.686 96.774) (end 156.21 98.298) (width 0.25) (layer B.Cu) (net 27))
 (segment (start 154.686 89.154) (end 154.686 96.774) (width 0.25) (layer B.Cu) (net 27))
 (segment (start 170.688 98.298) (end 156.21 98.298) (width 0.25) (layer B.Cu) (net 27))
 (segment (start 168.402 103.124) (end 168.402 107.442) (width 0.25) (layer B.Cu) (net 1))
 (segment (start 170.688 100.838) (end 168.402 103.124) (width 0.25) (layer B.Cu) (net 1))
 (via (at 168.402 107.442) (size 0.8) (drill 0.4) (layers F.Cu B.Cu) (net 1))
 (segment (start 168.402 107.442) (end 146.304 107.442) (width 0.25) (layer F.Cu) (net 1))
 (segment (start 146.304 107.442) (end 146.304 107.442) (width 0.25) (layer F.Cu) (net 1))
 (via (at 146.304 107.442) (size 0.8) (drill 0.4) (layers F.Cu B.Cu) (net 1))
 (segment (start 146.304 107.442) (end 146.304 101.6) (width 0.25) (layer B.Cu) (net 1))
 (segment (start 146.304 87.884) (end 146.304 85.598) (width 0.25) (layer B.Cu) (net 1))
 (via (at 146.304 87.884) (size 0.8) (drill 0.4) (layers F.Cu B.Cu) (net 1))
 (segment (start 146.304 85.598) (end 146.304 85.598) (width 0.25) (layer B.Cu) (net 1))
 (via (at 146.304 85.598) (size 0.8) (drill 0.4) (layers F.Cu B.Cu) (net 1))
 (segment (start 146.304 85.598) (end 147.828 85.598) (width 0.25) (layer F.Cu) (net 1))
 (segment (start 145.542 87.122) (end 146.304 87.884) (width 0.25) (layer F.Cu) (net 1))
 (segment (start 143.764 87.122) (end 145.542 87.122) (width 0.25) (layer F.Cu) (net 1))
 (segment (start 147.066 87.884) (end 147.828 88.646) (width 0.25) (layer F.Cu) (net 1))
 (segment (start 146.304 87.884) (end 147.066 87.884) (width 0.25) (layer F.Cu) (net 1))
 (segment (start 146.304 101.092) (end 146.304 87.884) (width 0.25) (layer B.Cu) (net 1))
 (segment (start 146.304 101.6) (end 146.304 101.092) (width 0.25) (layer B.Cu) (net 1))
 (via (at 146.304 101.6) (size 0.8) (drill 0.4) (layers F.Cu B.Cu) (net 1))
 (segment (start 138.43 101.6) (end 137.668 100.838) (width 0.25) (layer F.Cu) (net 1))
 (segment (start 146.304 101.6) (end 138.43 101.6) (width 0.25) (layer F.Cu) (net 1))
 (segment (start 163.576 88.9) (end 164.846 90.17) (width 0.25) (layer B.Cu) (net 28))
 (segment (start 163.576 86.614) (end 163.576 88.9) (width 0.25) (layer B.Cu) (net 28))
 (segment (start 151.384 105.664) (end 153.416 105.664) (width 0.25) (layer F.Cu) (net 4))
 (segment (start 153.416 105.664) (end 153.416 105.664) (width 0.25) (layer F.Cu) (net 4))
 (via (at 153.416 105.664) (size 0.8) (drill 0.4) (layers F.Cu B.Cu) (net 4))
 (segment (start 153.416 109.802) (end 153.596 109.982) (width 0.25) (layer B.Cu) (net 4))
 (segment (start 153.416 105.664) (end 153.416 109.802) (width 0.25) (layer B.Cu) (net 4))
 (segment (start 153.596 109.982) (end 147.828 109.982) (width 0.25) (layer F.Cu) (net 4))
 (segment (start 151.384 104.394) (end 158.242 104.394) (width 0.25) (layer F.Cu) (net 5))
 (segment (start 158.242 104.394) (end 158.242 104.394) (width 0.25) (layer F.Cu) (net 5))
 (via (at 158.242 104.394) (size 0.8) (drill 0.4) (layers F.Cu B.Cu) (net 5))
 (segment (start 158.242 109.728) (end 158.496 109.982) (width 0.25) (layer B.Cu) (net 5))
 (segment (start 158.242 104.394) (end 158.242 109.728) (width 0.25) (layer B.Cu) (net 5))
 (segment (start 158.496 109.982) (end 163.068 109.982) (width 0.25) (layer F.Cu) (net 5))
 (segment (start 145.542 99.822) (end 142.828 99.822) (width 0.25) (layer F.Cu) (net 6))
 (segment (start 146.812 98.552) (end 145.542 99.822) (width 0.25) (layer F.Cu) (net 6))
 (segment (start 149.098 98.552) (end 146.812 98.552) (width 0.25) (layer F.Cu) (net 6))
 (segment (start 149.86 99.314) (end 149.098 98.552) (width 0.25) (layer F.Cu) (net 6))
 (segment (start 151.384 99.314) (end 149.86 99.314) (width 0.25) (layer F.Cu) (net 6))
 (segment (start 155.956 88.392) (end 155.956 88.392) (width 0.25) (layer F.Cu) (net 7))
 (via (at 155.956 88.392) (size 0.8) (drill 0.4) (layers F.Cu B.Cu) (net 7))
 (segment (start 155.956 85.598) (end 155.956 88.392) (width 0.25) (layer B.Cu) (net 7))
 (segment (start 155.956 89.027) (end 155.956 88.392) (width 0.25) (layer F.Cu) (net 7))
 (segment (start 154.559 90.424) (end 155.956 89.027) (width 0.25) (layer F.Cu) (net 7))
 (segment (start 151.384 90.424) (end 154.559 90.424) (width 0.25) (layer F.Cu) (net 7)))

